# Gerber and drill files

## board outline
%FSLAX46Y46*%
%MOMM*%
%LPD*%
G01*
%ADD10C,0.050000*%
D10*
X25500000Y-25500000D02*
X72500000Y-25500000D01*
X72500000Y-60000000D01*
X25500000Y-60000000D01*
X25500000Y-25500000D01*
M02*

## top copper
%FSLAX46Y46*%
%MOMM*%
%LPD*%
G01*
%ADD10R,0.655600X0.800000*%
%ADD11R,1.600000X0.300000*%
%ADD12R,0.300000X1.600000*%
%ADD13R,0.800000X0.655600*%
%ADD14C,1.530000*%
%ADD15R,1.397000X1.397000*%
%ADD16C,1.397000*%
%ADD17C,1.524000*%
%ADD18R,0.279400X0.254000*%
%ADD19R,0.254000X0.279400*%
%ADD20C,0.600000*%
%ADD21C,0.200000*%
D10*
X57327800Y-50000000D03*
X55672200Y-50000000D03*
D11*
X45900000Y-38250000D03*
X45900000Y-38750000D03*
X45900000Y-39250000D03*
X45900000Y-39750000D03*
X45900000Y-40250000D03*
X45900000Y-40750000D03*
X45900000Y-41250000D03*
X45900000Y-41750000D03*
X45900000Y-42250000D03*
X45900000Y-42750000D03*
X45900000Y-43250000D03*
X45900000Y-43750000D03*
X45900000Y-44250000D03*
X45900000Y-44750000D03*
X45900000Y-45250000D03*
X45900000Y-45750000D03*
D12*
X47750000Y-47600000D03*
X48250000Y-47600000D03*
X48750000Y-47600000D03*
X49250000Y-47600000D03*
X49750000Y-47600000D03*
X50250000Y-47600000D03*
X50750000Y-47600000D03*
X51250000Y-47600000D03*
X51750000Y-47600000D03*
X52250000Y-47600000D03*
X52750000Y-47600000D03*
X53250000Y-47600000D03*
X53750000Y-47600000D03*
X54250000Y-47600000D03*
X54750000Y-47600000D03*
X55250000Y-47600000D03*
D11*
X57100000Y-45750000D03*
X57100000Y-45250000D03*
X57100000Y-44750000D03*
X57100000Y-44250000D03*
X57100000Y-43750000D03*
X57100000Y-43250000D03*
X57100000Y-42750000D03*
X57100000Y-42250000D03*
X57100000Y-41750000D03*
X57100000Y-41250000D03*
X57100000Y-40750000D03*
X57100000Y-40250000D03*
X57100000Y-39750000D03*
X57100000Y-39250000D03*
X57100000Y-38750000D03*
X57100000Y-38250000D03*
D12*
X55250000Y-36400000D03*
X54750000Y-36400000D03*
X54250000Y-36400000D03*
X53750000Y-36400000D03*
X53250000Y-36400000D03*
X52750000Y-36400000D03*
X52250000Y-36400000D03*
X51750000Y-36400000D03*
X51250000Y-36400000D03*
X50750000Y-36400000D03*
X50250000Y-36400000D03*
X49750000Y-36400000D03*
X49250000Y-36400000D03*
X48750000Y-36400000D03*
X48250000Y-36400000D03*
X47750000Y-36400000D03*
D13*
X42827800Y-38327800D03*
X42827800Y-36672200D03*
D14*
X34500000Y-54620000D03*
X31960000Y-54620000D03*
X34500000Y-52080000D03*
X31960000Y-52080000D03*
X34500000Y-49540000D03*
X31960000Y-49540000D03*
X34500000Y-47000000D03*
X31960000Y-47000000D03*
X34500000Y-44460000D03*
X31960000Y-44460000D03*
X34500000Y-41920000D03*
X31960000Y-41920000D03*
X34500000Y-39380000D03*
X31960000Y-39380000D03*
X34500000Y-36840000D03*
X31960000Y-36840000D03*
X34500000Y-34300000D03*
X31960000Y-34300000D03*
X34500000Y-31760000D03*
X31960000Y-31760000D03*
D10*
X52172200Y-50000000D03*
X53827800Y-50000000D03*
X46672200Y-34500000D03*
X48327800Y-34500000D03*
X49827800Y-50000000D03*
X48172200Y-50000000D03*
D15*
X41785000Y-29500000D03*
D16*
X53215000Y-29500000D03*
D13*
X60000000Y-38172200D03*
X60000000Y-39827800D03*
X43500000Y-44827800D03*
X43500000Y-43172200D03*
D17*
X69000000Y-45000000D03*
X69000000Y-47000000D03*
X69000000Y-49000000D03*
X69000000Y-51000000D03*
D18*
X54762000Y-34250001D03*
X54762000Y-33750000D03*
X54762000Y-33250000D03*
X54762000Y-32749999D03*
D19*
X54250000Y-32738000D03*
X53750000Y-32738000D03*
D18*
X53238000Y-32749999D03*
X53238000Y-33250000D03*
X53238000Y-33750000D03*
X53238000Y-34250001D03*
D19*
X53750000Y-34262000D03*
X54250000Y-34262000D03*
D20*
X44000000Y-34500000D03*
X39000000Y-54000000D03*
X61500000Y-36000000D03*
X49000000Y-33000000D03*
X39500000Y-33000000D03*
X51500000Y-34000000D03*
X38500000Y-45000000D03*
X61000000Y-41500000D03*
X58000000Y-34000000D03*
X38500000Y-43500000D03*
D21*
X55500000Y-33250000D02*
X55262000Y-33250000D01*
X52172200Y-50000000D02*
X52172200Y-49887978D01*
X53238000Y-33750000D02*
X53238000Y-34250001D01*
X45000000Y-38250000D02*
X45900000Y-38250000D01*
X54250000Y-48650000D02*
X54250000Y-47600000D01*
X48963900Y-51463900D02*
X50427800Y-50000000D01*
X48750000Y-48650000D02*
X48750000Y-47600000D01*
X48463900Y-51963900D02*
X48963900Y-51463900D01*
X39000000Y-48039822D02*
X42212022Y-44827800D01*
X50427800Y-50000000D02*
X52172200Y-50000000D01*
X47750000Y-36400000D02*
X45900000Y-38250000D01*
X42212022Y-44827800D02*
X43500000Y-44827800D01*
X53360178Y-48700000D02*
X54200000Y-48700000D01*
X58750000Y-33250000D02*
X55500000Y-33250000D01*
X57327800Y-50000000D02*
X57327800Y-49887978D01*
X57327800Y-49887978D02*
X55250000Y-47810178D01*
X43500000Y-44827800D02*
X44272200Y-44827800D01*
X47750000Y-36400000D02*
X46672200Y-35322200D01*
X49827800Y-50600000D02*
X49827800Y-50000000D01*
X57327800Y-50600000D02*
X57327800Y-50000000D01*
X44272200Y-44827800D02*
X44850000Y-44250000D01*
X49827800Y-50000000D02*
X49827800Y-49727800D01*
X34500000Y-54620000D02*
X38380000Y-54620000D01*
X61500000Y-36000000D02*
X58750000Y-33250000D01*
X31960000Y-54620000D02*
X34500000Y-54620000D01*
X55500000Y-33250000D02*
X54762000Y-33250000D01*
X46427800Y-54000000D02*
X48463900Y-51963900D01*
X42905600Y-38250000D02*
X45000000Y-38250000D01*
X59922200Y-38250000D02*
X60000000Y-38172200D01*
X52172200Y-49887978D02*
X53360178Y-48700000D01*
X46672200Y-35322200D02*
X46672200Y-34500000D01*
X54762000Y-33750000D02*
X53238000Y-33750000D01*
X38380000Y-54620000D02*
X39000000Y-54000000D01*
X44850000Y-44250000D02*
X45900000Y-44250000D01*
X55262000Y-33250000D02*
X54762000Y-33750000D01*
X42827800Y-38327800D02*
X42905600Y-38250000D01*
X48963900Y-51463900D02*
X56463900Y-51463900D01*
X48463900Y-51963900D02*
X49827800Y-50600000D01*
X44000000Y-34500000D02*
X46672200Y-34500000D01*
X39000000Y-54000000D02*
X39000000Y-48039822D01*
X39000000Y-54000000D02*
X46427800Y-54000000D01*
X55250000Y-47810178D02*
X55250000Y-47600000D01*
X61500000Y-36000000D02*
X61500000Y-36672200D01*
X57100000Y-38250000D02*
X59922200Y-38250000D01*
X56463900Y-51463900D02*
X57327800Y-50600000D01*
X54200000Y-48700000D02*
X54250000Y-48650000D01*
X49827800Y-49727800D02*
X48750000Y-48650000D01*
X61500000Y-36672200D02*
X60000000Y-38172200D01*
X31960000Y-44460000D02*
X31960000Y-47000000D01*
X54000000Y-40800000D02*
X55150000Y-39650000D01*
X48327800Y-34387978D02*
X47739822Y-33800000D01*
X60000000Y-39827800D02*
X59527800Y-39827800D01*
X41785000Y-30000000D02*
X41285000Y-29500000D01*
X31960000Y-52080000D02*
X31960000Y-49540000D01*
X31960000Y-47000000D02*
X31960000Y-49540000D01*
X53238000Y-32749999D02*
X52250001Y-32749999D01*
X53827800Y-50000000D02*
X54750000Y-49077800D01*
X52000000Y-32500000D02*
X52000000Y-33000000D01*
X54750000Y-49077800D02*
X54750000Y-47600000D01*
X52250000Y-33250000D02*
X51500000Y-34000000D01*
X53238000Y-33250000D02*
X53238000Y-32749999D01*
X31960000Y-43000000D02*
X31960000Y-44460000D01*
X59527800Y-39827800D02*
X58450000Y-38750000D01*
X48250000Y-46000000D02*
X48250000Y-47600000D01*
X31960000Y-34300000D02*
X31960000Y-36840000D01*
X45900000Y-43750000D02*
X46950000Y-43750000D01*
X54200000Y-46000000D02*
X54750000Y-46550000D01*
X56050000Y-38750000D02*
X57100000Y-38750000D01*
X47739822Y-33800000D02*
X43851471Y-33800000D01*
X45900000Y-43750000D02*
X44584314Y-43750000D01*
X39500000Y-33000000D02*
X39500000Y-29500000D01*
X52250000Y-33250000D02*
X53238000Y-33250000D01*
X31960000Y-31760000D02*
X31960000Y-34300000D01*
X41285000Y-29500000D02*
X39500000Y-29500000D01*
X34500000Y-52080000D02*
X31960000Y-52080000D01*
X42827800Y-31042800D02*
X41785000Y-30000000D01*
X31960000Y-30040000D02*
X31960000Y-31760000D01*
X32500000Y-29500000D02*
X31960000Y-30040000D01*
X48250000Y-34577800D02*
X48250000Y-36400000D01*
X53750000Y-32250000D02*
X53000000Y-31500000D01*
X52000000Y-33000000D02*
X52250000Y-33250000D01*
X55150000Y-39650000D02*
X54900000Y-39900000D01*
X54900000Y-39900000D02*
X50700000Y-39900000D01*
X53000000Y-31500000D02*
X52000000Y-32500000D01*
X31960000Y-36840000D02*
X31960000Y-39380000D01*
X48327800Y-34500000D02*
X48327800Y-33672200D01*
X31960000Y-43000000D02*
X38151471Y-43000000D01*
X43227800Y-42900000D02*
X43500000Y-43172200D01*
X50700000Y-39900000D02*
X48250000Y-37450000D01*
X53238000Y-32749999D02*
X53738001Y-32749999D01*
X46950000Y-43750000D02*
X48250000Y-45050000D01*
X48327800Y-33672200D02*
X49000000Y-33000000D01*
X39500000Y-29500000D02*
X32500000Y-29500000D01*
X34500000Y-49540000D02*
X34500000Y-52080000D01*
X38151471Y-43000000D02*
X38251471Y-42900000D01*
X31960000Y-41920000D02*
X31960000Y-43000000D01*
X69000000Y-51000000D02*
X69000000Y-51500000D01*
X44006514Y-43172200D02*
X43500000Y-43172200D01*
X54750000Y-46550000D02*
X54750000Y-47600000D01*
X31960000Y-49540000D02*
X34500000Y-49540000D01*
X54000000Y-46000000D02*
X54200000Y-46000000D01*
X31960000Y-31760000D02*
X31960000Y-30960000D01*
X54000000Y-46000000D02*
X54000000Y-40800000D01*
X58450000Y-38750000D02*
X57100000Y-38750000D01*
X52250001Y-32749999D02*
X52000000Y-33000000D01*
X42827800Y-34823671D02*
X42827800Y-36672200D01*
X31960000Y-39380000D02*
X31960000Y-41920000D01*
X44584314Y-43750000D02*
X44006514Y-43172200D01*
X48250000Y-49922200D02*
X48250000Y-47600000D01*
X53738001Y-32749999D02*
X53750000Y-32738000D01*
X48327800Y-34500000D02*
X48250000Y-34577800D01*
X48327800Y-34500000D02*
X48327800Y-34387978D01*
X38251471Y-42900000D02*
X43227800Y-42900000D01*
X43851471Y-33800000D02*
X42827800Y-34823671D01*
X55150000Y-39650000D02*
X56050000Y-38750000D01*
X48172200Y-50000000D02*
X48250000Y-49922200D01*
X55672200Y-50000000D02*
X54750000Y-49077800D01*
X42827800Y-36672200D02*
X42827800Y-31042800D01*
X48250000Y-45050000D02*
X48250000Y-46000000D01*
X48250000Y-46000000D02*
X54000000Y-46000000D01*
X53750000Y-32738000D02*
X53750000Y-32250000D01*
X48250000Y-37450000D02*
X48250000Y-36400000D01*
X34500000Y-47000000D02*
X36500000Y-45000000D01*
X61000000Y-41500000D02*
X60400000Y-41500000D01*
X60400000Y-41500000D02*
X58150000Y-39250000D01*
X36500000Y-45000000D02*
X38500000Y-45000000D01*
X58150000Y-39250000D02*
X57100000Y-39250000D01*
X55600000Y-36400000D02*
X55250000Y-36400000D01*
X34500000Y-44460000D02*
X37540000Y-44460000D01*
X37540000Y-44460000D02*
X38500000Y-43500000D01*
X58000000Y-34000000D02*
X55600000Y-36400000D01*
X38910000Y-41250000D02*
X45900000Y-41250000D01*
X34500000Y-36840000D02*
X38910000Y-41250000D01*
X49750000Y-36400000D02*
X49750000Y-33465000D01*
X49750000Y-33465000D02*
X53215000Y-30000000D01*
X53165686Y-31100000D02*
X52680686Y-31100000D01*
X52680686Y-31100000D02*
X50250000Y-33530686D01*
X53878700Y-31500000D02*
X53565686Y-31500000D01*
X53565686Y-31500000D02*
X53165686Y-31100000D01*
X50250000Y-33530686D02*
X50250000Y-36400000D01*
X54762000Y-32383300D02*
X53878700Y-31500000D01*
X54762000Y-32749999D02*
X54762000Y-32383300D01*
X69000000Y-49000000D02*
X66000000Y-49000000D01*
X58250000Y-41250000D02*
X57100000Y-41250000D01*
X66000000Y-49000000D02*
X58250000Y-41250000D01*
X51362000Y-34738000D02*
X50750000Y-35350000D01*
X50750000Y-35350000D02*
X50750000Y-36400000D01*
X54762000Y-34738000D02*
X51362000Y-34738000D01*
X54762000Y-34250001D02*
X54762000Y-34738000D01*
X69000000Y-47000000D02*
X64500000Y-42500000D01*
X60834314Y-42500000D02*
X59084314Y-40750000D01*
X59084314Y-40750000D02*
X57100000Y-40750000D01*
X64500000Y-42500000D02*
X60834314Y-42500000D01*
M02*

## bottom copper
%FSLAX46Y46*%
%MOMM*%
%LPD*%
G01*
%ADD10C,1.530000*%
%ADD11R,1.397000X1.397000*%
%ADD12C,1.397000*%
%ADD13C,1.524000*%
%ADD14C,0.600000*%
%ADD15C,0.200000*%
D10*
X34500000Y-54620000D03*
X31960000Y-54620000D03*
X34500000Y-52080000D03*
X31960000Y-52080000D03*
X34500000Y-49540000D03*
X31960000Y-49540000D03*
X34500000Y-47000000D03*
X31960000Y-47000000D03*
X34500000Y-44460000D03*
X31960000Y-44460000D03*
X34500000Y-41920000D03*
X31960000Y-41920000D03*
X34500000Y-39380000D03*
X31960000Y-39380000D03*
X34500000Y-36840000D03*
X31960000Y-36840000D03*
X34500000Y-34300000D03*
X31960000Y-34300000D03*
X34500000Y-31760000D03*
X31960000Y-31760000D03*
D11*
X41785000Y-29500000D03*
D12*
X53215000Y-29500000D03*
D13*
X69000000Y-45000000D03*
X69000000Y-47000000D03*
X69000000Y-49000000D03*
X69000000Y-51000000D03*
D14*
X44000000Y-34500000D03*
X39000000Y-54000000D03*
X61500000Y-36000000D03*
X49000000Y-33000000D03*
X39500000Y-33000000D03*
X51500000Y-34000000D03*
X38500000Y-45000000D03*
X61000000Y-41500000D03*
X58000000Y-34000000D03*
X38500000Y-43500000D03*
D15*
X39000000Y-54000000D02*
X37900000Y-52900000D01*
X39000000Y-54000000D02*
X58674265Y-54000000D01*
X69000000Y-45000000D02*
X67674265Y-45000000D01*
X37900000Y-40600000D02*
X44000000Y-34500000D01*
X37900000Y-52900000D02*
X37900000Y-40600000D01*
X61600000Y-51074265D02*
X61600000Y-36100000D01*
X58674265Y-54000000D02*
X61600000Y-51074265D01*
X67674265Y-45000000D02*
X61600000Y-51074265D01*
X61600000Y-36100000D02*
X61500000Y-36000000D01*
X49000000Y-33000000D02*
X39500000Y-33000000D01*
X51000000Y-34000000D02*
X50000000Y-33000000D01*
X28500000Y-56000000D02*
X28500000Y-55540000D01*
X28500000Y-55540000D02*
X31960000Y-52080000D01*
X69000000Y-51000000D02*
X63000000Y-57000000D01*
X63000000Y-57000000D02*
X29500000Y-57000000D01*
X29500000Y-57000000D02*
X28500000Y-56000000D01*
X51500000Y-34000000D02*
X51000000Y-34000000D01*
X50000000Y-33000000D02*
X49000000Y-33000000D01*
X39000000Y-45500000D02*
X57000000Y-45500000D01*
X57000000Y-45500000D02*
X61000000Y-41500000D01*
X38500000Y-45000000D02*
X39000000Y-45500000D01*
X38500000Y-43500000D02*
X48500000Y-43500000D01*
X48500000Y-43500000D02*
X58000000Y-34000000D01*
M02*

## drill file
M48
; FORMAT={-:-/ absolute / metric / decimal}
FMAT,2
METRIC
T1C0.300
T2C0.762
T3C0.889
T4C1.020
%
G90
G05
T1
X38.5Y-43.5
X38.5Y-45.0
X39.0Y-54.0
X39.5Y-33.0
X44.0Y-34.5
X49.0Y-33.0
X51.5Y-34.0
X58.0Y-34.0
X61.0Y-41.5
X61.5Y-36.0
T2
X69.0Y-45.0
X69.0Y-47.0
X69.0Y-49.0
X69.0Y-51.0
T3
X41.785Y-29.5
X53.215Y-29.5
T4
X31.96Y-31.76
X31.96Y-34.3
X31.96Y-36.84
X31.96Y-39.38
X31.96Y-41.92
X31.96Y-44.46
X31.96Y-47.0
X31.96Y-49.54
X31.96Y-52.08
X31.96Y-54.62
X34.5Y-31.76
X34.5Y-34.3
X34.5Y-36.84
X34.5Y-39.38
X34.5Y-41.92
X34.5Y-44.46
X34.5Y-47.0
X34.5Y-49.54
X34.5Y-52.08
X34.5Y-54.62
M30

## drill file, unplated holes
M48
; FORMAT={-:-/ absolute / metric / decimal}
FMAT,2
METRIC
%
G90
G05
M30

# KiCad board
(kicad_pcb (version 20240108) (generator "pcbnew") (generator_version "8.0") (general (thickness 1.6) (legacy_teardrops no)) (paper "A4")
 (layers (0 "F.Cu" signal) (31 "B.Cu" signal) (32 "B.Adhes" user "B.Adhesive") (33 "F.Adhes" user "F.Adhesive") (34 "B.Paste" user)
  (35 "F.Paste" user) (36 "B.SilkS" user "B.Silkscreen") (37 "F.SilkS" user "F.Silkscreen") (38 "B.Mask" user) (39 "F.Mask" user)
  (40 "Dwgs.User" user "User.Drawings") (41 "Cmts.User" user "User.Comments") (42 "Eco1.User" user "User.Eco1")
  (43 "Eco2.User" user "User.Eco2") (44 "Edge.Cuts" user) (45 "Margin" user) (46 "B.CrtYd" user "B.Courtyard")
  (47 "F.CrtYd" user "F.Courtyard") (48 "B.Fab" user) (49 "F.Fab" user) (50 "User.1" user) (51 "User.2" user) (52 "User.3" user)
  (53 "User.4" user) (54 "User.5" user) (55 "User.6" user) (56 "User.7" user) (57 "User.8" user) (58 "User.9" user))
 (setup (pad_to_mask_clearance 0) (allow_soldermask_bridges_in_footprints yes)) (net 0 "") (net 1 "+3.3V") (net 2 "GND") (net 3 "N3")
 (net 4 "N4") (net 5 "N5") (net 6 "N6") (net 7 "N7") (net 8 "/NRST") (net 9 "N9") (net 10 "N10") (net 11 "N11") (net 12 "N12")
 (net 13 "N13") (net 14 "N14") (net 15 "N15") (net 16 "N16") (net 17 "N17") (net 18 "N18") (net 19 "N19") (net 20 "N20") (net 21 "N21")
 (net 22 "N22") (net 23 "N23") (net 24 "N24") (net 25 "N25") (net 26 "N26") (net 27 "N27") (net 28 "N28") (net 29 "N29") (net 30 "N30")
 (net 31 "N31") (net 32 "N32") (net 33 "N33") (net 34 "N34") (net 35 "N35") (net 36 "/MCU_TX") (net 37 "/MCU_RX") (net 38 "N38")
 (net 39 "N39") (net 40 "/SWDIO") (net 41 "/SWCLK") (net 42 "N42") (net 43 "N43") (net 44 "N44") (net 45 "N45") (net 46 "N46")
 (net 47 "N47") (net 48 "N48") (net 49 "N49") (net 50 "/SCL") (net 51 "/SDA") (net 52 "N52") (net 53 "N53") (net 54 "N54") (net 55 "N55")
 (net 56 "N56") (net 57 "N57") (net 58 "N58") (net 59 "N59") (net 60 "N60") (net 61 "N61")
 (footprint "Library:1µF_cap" (layer "F.Cu") (at 56.5 50 180)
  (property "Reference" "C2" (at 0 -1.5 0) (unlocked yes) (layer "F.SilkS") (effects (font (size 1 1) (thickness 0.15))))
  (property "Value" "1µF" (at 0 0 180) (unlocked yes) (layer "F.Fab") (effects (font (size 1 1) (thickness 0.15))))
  (pad "1" smd rect (at -0.8278 0 180) (size 0.6556 0.8) (layers "F.Cu" "F.Paste" "F.Mask") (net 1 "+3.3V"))
  (pad "2" smd rect (at 0.8278 0 180) (size 0.6556 0.8) (layers "F.Cu" "F.Paste" "F.Mask") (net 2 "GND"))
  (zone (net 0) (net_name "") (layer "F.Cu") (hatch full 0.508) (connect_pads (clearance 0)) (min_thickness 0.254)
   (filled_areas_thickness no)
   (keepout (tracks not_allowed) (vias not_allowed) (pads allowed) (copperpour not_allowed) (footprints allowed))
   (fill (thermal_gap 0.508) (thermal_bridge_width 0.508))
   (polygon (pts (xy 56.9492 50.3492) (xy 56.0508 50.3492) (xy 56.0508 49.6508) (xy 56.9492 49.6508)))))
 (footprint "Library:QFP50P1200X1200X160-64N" (layer "F.Cu") (at 51.5 42)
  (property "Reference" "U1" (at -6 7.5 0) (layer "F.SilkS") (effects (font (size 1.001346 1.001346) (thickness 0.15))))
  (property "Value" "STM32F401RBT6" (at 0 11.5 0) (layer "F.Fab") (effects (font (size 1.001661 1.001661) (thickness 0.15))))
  (pad "1" smd rect (at -5.6 -3.75) (size 1.6 0.3) (layers "F.Cu" "F.Paste" "F.Mask") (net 1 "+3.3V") (solder_mask_margin 0.102))
  (pad "2" smd rect (at -5.6 -3.25) (size 1.6 0.3) (layers "F.Cu" "F.Paste" "F.Mask") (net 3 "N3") (solder_mask_margin 0.102))
  (pad "3" smd rect (at -5.6 -2.75) (size 1.6 0.3) (layers "F.Cu" "F.Paste" "F.Mask") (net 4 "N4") (solder_mask_margin 0.102))
  (pad "4" smd rect (at -5.6 -2.25) (size 1.6 0.3) (layers "F.Cu" "F.Paste" "F.Mask") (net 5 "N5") (solder_mask_margin 0.102))
  (pad "5" smd rect (at -5.6 -1.75) (size 1.6 0.3) (layers "F.Cu" "F.Paste" "F.Mask") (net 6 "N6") (solder_mask_margin 0.102))
  (pad "6" smd rect (at -5.6 -1.25) (size 1.6 0.3) (layers "F.Cu" "F.Paste" "F.Mask") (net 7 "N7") (solder_mask_margin 0.102))
  (pad "7" smd rect (at -5.6 -0.75) (size 1.6 0.3) (layers "F.Cu" "F.Paste" "F.Mask") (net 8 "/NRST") (solder_mask_margin 0.102))
  (pad "8" smd rect (at -5.6 -0.25) (size 1.6 0.3) (layers "F.Cu" "F.Paste" "F.Mask") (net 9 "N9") (solder_mask_margin 0.102))
  (pad "9" smd rect (at -5.6 0.25) (size 1.6 0.3) (layers "F.Cu" "F.Paste" "F.Mask") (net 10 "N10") (solder_mask_margin 0.102))
  (pad "10" smd rect (at -5.6 0.75) (size 1.6 0.3) (layers "F.Cu" "F.Paste" "F.Mask") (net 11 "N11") (solder_mask_margin 0.102))
  (pad "11" smd rect (at -5.6 1.25) (size 1.6 0.3) (layers "F.Cu" "F.Paste" "F.Mask") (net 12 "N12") (solder_mask_margin 0.102))
  (pad "12" smd rect (at -5.6 1.75) (size 1.6 0.3) (layers "F.Cu" "F.Paste" "F.Mask") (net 2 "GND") (solder_mask_margin 0.102))
  (pad "13" smd rect (at -5.6 2.25) (size 1.6 0.3) (layers "F.Cu" "F.Paste" "F.Mask") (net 1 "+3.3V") (solder_mask_margin 0.102))
  (pad "14" smd rect (at -5.6 2.75) (size 1.6 0.3) (layers "F.Cu" "F.Paste" "F.Mask") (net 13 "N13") (solder_mask_margin 0.102))
  (pad "15" smd rect (at -5.6 3.25) (size 1.6 0.3) (layers "F.Cu" "F.Paste" "F.Mask") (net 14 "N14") (solder_mask_margin 0.102))
  (pad "16" smd rect (at -5.6 3.75) (size 1.6 0.3) (layers "F.Cu" "F.Paste" "F.Mask") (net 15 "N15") (solder_mask_margin 0.102))
  (pad "17" smd rect (at -3.75 5.6) (size 0.3 1.6) (layers "F.Cu" "F.Paste" "F.Mask") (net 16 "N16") (solder_mask_margin 0.102))
  (pad "18" smd rect (at -3.25 5.6) (size 0.3 1.6) (layers "F.Cu" "F.Paste" "F.Mask") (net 2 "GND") (solder_mask_margin 0.102))
  (pad "19" smd rect (at -2.75 5.6) (size 0.3 1.6) (layers "F.Cu" "F.Paste" "F.Mask") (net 1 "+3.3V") (solder_mask_margin 0.102))
  (pad "20" smd rect (at -2.25 5.6) (size 0.3 1.6) (layers "F.Cu" "F.Paste" "F.Mask") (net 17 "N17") (solder_mask_margin 0.102))
  (pad "21" smd rect (at -1.75 5.6) (size 0.3 1.6) (layers "F.Cu" "F.Paste" "F.Mask") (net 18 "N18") (solder_mask_margin 0.102))
  (pad "22" smd rect (at -1.25 5.6) (size 0.3 1.6) (layers "F.Cu" "F.Paste" "F.Mask") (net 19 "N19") (solder_mask_margin 0.102))
  (pad "23" smd rect (at -0.75 5.6) (size 0.3 1.6) (layers "F.Cu" "F.Paste" "F.Mask") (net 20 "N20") (solder_mask_margin 0.102))
  (pad "24" smd rect (at -0.25 5.6) (size 0.3 1.6) (layers "F.Cu" "F.Paste" "F.Mask") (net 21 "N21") (solder_mask_margin 0.102))
  (pad "25" smd rect (at 0.25 5.6) (size 0.3 1.6) (layers "F.Cu" "F.Paste" "F.Mask") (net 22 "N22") (solder_mask_margin 0.102))
  (pad "26" smd rect (at 0.75 5.6) (size 0.3 1.6) (layers "F.Cu" "F.Paste" "F.Mask") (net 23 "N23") (solder_mask_margin 0.102))
  (pad "27" smd rect (at 1.25 5.6) (size 0.3 1.6) (layers "F.Cu" "F.Paste" "F.Mask") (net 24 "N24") (solder_mask_margin 0.102))
  (pad "28" smd rect (at 1.75 5.6) (size 0.3 1.6) (layers "F.Cu" "F.Paste" "F.Mask") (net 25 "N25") (solder_mask_margin 0.102))
  (pad "29" smd rect (at 2.25 5.6) (size 0.3 1.6) (layers "F.Cu" "F.Paste" "F.Mask") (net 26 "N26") (solder_mask_margin 0.102))
  (pad "30" smd rect (at 2.75 5.6) (size 0.3 1.6) (layers "F.Cu" "F.Paste" "F.Mask") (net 1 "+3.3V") (solder_mask_margin 0.102))
  (pad "31" smd rect (at 3.25 5.6) (size 0.3 1.6) (layers "F.Cu" "F.Paste" "F.Mask") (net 2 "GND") (solder_mask_margin 0.102))
  (pad "32" smd rect (at 3.75 5.6) (size 0.3 1.6) (layers "F.Cu" "F.Paste" "F.Mask") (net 1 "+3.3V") (solder_mask_margin 0.102))
  (pad "33" smd rect (at 5.6 3.75) (size 1.6 0.3) (layers "F.Cu" "F.Paste" "F.Mask") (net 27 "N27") (solder_mask_margin 0.102))
  (pad "34" smd rect (at 5.6 3.25) (size 1.6 0.3) (layers "F.Cu" "F.Paste" "F.Mask") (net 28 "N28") (solder_mask_margin 0.102))
  (pad "35" smd rect (at 5.6 2.75) (size 1.6 0.3) (layers "F.Cu" "F.Paste" "F.Mask") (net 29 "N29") (solder_mask_margin 0.102))
  (pad "36" smd rect (at 5.6 2.25) (size 1.6 0.3) (layers "F.Cu" "F.Paste" "F.Mask") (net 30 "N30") (solder_mask_margin 0.102))
  (pad "37" smd rect (at 5.6 1.75) (size 1.6 0.3) (layers "F.Cu" "F.Paste" "F.Mask") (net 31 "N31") (solder_mask_margin 0.102))
  (pad "38" smd rect (at 5.6 1.25) (size 1.6 0.3) (layers "F.Cu" "F.Paste" "F.Mask") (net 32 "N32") (solder_mask_margin 0.102))
  (pad "39" smd rect (at 5.6 0.75) (size 1.6 0.3) (layers "F.Cu" "F.Paste" "F.Mask") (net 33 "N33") (solder_mask_margin 0.102))
  (pad "40" smd rect (at 5.6 0.25) (size 1.6 0.3) (layers "F.Cu" "F.Paste" "F.Mask") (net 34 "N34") (solder_mask_margin 0.102))
  (pad "41" smd rect (at 5.6 -0.25) (size 1.6 0.3) (layers "F.Cu" "F.Paste" "F.Mask") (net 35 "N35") (solder_mask_margin 0.102))
  (pad "42" smd rect (at 5.6 -0.75) (size 1.6 0.3) (layers "F.Cu" "F.Paste" "F.Mask") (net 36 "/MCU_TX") (solder_mask_margin 0.102))
  (pad "43" smd rect (at 5.6 -1.25) (size 1.6 0.3) (layers "F.Cu" "F.Paste" "F.Mask") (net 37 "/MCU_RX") (solder_mask_margin 0.102))
  (pad "44" smd rect (at 5.6 -1.75) (size 1.6 0.3) (layers "F.Cu" "F.Paste" "F.Mask") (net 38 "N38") (solder_mask_margin 0.102))
  (pad "45" smd rect (at 5.6 -2.25) (size 1.6 0.3) (layers "F.Cu" "F.Paste" "F.Mask") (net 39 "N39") (solder_mask_margin 0.102))
  (pad "46" smd rect (at 5.6 -2.75) (size 1.6 0.3) (layers "F.Cu" "F.Paste" "F.Mask") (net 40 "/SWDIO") (solder_mask_margin 0.102))
  (pad "47" smd rect (at 5.6 -3.25) (size 1.6 0.3) (layers "F.Cu" "F.Paste" "F.Mask") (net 2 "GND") (solder_mask_margin 0.102))
  (pad "48" smd rect (at 5.6 -3.75) (size 1.6 0.3) (layers "F.Cu" "F.Paste" "F.Mask") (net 1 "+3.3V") (solder_mask_margin 0.102))
  (pad "49" smd rect (at 3.75 -5.6) (size 0.3 1.6) (layers "F.Cu" "F.Paste" "F.Mask") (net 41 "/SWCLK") (solder_mask_margin 0.102))
  (pad "50" smd rect (at 3.25 -5.6) (size 0.3 1.6) (layers "F.Cu" "F.Paste" "F.Mask") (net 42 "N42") (solder_mask_margin 0.102))
  (pad "51" smd rect (at 2.75 -5.6) (size 0.3 1.6) (layers "F.Cu" "F.Paste" "F.Mask") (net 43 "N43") (solder_mask_margin 0.102))
  (pad "52" smd rect (at 2.25 -5.6) (size 0.3 1.6) (layers "F.Cu" "F.Paste" "F.Mask") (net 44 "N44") (solder_mask_margin 0.102))
  (pad "53" smd rect (at 1.75 -5.6) (size 0.3 1.6) (layers "F.Cu" "F.Paste" "F.Mask") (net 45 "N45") (solder_mask_margin 0.102))
  (pad "54" smd rect (at 1.25 -5.6) (size 0.3 1.6) (layers "F.Cu" "F.Paste" "F.Mask") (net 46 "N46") (solder_mask_margin 0.102))
  (pad "55" smd rect (at 0.75 -5.6) (size 0.3 1.6) (layers "F.Cu" "F.Paste" "F.Mask") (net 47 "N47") (solder_mask_margin 0.102))
  (pad "56" smd rect (at 0.25 -5.6) (size 0.3 1.6) (layers "F.Cu" "F.Paste" "F.Mask") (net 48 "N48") (solder_mask_margin 0.102))
  (pad "57" smd rect (at -0.25 -5.6) (size 0.3 1.6) (layers "F.Cu" "F.Paste" "F.Mask") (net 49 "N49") (solder_mask_margin 0.102))
  (pad "58" smd rect (at -0.75 -5.6) (size 0.3 1.6) (layers "F.Cu" "F.Paste" "F.Mask") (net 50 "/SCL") (solder_mask_margin 0.102))
  (pad "59" smd rect (at -1.25 -5.6) (size 0.3 1.6) (layers "F.Cu" "F.Paste" "F.Mask") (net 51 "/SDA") (solder_mask_margin 0.102))
  (pad "60" smd rect (at -1.75 -5.6) (size 0.3 1.6) (layers "F.Cu" "F.Paste" "F.Mask") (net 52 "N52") (solder_mask_margin 0.102))
  (pad "61" smd rect (at -2.25 -5.6) (size 0.3 1.6) (layers "F.Cu" "F.Paste" "F.Mask") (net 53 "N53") (solder_mask_margin 0.102))
  (pad "62" smd rect (at -2.75 -5.6) (size 0.3 1.6) (layers "F.Cu" "F.Paste" "F.Mask") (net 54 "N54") (solder_mask_margin 0.102))
  (pad "63" smd rect (at -3.25 -5.6) (size 0.3 1.6) (layers "F.Cu" "F.Paste" "F.Mask") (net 2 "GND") (solder_mask_margin 0.102))
  (pad "64" smd rect (at -3.75 -5.6) (size 0.3 1.6) (layers "F.Cu" "F.Paste" "F.Mask") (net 1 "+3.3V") (solder_mask_margin 0.102)))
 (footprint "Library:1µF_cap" (layer "F.Cu") (at 42.8278 37.5 90)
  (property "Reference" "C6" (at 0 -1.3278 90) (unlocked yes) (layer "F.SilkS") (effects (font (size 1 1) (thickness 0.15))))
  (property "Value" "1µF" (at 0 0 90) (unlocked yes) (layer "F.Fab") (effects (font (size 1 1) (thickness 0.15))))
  (pad "1" smd rect (at -0.8278 0 90) (size 0.6556 0.8) (layers "F.Cu" "F.Paste" "F.Mask") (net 1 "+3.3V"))
  (pad "2" smd rect (at 0.8278 0 90) (size 0.6556 0.8) (layers "F.Cu" "F.Paste" "F.Mask") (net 2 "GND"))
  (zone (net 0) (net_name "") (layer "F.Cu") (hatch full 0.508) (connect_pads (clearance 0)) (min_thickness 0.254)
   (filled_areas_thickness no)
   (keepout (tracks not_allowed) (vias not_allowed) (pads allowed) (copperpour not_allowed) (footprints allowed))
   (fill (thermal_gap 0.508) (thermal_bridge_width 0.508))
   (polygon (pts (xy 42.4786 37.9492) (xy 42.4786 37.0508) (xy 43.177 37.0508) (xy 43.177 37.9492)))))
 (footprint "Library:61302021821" (layer "F.Cu") (at 33.23 43.19 90)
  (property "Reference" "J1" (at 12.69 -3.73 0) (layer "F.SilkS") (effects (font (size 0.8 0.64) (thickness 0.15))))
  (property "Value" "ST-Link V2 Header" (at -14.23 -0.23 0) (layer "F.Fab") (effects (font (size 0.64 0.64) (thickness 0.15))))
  (pad "1" thru_hole circle (at -11.43 1.27 90) (size 1.53 1.53) (drill 1.02) (layers "*.Cu" "*.Mask") (remove_unused_layers no)
   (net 1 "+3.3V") (solder_mask_margin 0.102))
  (pad "2" thru_hole circle (at -11.43 -1.27 90) (size 1.53 1.53) (drill 1.02) (layers "*.Cu" "*.Mask") (remove_unused_layers no)
   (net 1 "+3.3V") (solder_mask_margin 0.102))
  (pad "3" thru_hole circle (at -8.89 1.27 90) (size 1.53 1.53) (drill 1.02) (layers "*.Cu" "*.Mask") (remove_unused_layers no)
   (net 2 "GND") (solder_mask_margin 0.102))
  (pad "4" thru_hole circle (at -8.89 -1.27 90) (size 1.53 1.53) (drill 1.02) (layers "*.Cu" "*.Mask") (remove_unused_layers no)
   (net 2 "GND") (solder_mask_margin 0.102))
  (pad "5" thru_hole circle (at -6.35 1.27 90) (size 1.53 1.53) (drill 1.02) (layers "*.Cu" "*.Mask") (remove_unused_layers no)
   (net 2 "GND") (solder_mask_margin 0.102))
  (pad "6" thru_hole circle (at -6.35 -1.27 90) (size 1.53 1.53) (drill 1.02) (layers "*.Cu" "*.Mask") (remove_unused_layers no)
   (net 2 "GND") (solder_mask_margin 0.102))
  (pad "7" thru_hole circle (at -3.81 1.27 90) (size 1.53 1.53) (drill 1.02) (layers "*.Cu" "*.Mask") (remove_unused_layers no)
   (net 40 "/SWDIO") (solder_mask_margin 0.102))
  (pad "8" thru_hole circle (at -3.81 -1.27 90) (size 1.53 1.53) (drill 1.02) (layers "*.Cu" "*.Mask") (remove_unused_layers no)
   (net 2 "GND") (solder_mask_margin 0.102))
  (pad "9" thru_hole circle (at -1.27 1.27 90) (size 1.53 1.53) (drill 1.02) (layers "*.Cu" "*.Mask") (remove_unused_layers no)
   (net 41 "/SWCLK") (solder_mask_margin 0.102))
  (pad "10" thru_hole circle (at -1.27 -1.27 90) (size 1.53 1.53) (drill 1.02) (layers "*.Cu" "*.Mask") (remove_unused_layers no)
   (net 2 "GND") (solder_mask_margin 0.102))
  (pad "11" thru_hole circle (at 1.27 1.27 90) (size 1.53 1.53) (drill 1.02) (layers "*.Cu" "*.Mask") (remove_unused_layers no)
   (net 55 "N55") (solder_mask_margin 0.102))
  (pad "12" thru_hole circle (at 1.27 -1.27 90) (size 1.53 1.53) (drill 1.02) (layers "*.Cu" "*.Mask") (remove_unused_layers no)
   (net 2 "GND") (solder_mask_margin 0.102))
  (pad "13" thru_hole circle (at 3.81 1.27 90) (size 1.53 1.53) (drill 1.02) (layers "*.Cu" "*.Mask") (remove_unused_layers no)
   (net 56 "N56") (solder_mask_margin 0.102))
  (pad "14" thru_hole circle (at 3.81 -1.27 90) (size 1.53 1.53) (drill 1.02) (layers "*.Cu" "*.Mask") (remove_unused_layers no)
   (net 2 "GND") (solder_mask_margin 0.102))
  (pad "15" thru_hole circle (at 6.35 1.27 90) (size 1.53 1.53) (drill 1.02) (layers "*.Cu" "*.Mask") (remove_unused_layers no)
   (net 8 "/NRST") (solder_mask_margin 0.102))
  (pad "16" thru_hole circle (at 6.35 -1.27 90) (size 1.53 1.53) (drill 1.02) (layers "*.Cu" "*.Mask") (remove_unused_layers no)
   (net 2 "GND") (solder_mask_margin 0.102))
  (pad "17" thru_hole circle (at 8.89 1.27 90) (size 1.53 1.53) (drill 1.02) (layers "*.Cu" "*.Mask") (remove_unused_layers no)
   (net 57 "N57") (solder_mask_margin 0.102))
  (pad "18" thru_hole circle (at 8.89 -1.27 90) (size 1.53 1.53) (drill 1.02) (layers "*.Cu" "*.Mask") (remove_unused_layers no)
   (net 2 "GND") (solder_mask_margin 0.102))
  (pad "19" thru_hole circle (at 11.43 1.27 90) (size 1.53 1.53) (drill 1.02) (layers "*.Cu" "*.Mask") (remove_unused_layers no)
   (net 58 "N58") (solder_mask_margin 0.102))
  (pad "20" thru_hole circle (at 11.43 -1.27 90) (size 1.53 1.53) (drill 1.02) (layers "*.Cu" "*.Mask") (remove_unused_layers no)
   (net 2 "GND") (solder_mask_margin 0.102)))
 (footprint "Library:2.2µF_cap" (layer "F.Cu") (at 53 50)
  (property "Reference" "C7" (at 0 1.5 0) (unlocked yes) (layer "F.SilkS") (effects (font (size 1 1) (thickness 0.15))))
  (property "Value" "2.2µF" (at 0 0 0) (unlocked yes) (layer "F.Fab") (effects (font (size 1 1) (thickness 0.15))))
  (pad "1" smd rect (at -0.8278 0) (size 0.6556 0.8) (layers "F.Cu" "F.Paste" "F.Mask") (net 1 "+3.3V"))
  (pad "2" smd rect (at 0.8278 0) (size 0.6556 0.8) (layers "F.Cu" "F.Paste" "F.Mask") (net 2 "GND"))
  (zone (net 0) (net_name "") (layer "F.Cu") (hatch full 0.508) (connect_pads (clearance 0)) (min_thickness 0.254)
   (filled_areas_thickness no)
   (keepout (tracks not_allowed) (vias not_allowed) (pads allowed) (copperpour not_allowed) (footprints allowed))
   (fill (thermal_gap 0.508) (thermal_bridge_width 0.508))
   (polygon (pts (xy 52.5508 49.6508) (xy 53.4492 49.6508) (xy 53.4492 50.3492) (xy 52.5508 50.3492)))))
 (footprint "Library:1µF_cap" (layer "F.Cu") (at 47.5 34.5)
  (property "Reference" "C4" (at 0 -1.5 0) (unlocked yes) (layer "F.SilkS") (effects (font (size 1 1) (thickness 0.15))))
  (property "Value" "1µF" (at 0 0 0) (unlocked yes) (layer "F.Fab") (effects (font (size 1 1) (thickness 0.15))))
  (pad "1" smd rect (at -0.8278 0) (size 0.6556 0.8) (layers "F.Cu" "F.Paste" "F.Mask") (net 1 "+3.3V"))
  (pad "2" smd rect (at 0.8278 0) (size 0.6556 0.8) (layers "F.Cu" "F.Paste" "F.Mask") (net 2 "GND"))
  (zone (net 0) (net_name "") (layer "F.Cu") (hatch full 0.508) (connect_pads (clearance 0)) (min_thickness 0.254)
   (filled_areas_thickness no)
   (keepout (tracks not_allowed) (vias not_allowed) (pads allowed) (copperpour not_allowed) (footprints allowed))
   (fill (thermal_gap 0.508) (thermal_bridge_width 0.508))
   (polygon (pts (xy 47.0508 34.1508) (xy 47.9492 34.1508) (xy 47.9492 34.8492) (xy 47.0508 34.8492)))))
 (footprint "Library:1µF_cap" (layer "F.Cu") (at 49 50 180)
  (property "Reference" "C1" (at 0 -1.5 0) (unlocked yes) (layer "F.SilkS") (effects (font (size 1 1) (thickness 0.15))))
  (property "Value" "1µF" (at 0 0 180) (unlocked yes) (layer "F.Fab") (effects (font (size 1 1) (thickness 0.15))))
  (pad "1" smd rect (at -0.8278 0 180) (size 0.6556 0.8) (layers "F.Cu" "F.Paste" "F.Mask") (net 1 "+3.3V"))
  (pad "2" smd rect (at 0.8278 0 180) (size 0.6556 0.8) (layers "F.Cu" "F.Paste" "F.Mask") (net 2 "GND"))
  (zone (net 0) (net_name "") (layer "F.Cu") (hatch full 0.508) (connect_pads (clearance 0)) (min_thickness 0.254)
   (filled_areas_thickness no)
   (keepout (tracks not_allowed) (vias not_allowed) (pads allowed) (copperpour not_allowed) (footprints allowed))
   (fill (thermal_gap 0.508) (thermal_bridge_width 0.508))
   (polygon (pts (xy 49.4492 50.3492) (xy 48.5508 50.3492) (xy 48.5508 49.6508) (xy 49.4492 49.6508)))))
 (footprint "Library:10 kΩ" (layer "F.Cu") (at 41.785 29.5)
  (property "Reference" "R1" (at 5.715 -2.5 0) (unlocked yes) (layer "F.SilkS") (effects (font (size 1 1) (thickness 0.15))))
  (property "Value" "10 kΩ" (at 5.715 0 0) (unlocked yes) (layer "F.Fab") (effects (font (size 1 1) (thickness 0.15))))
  (pad "1" thru_hole rect (at 0 0) (size 1.397 1.397) (drill 0.889) (layers "*.Cu" "*.Mask") (remove_unused_layers no) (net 2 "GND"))
  (pad "2" thru_hole circle (at 11.43 0) (size 1.397 1.397) (drill 0.889) (layers "*.Cu" "*.Mask") (remove_unused_layers no) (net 52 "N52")))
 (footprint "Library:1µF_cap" (layer "F.Cu") (at 60 39 -90)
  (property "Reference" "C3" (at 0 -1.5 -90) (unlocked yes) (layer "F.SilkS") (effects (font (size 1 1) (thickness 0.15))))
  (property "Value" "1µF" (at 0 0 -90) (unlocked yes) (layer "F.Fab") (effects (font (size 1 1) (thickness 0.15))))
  (pad "1" smd rect (at -0.8278 0 270) (size 0.6556 0.8) (layers "F.Cu" "F.Paste" "F.Mask") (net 1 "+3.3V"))
  (pad "2" smd rect (at 0.8278 0 270) (size 0.6556 0.8) (layers "F.Cu" "F.Paste" "F.Mask") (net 2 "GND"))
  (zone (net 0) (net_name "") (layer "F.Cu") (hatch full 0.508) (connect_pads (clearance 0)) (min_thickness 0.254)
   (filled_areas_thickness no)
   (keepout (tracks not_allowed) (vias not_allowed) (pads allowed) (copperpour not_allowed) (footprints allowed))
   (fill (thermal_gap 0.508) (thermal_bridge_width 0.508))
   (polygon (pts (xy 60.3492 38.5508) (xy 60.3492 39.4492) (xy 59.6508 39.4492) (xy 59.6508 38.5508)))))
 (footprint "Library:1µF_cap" (layer "F.Cu") (at 43.5 44 90)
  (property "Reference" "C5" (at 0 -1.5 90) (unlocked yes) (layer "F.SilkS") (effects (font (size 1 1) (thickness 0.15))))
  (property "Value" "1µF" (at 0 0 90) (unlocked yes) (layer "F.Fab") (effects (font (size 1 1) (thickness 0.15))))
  (pad "1" smd rect (at -0.8278 0 90) (size 0.6556 0.8) (layers "F.Cu" "F.Paste" "F.Mask") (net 1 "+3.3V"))
  (pad "2" smd rect (at 0.8278 0 90) (size 0.6556 0.8) (layers "F.Cu" "F.Paste" "F.Mask") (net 2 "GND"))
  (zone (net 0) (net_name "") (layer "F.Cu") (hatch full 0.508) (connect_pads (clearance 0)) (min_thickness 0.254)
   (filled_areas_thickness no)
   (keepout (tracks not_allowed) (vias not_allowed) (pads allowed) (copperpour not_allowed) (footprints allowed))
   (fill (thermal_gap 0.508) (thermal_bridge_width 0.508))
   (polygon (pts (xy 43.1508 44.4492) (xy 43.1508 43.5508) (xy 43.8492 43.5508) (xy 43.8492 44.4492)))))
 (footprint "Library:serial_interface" (layer "F.Cu") (at 69 48 -90)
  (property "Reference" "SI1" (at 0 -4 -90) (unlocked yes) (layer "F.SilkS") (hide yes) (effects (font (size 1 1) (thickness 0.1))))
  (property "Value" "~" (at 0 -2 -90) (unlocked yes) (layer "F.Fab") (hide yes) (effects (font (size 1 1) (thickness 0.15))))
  (pad "1" thru_hole circle (at -3 0 270) (size 1.524 1.524) (drill 0.762) (layers "*.Cu" "*.Mask") (remove_unused_layers no)
   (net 1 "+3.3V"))
  (pad "2" thru_hole circle (at -1 0 270) (size 1.524 1.524) (drill 0.762) (layers "*.Cu" "*.Mask") (remove_unused_layers no)
   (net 37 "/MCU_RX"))
  (pad "3" thru_hole circle (at 1 0 270) (size 1.524 1.524) (drill 0.762) (layers "*.Cu" "*.Mask") (remove_unused_layers no)
   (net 36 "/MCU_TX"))
  (pad "4" thru_hole circle (at 3 0 270) (size 1.524 1.524) (drill 0.762) (layers "*.Cu" "*.Mask") (remove_unused_layers no) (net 2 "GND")))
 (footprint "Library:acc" (layer "F.Cu") (at 54 33.5 180)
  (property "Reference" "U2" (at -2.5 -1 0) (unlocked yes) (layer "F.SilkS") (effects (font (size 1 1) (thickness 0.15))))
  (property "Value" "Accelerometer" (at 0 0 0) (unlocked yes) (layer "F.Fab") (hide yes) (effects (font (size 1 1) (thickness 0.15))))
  (pad "1" smd rect (at -0.762 -0.750001 270) (size 0.254 0.2794) (layers "F.Cu" "F.Paste" "F.Mask") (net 50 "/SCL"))
  (pad "2" smd rect (at -0.762 -0.25 270) (size 0.254 0.2794) (layers "F.Cu" "F.Paste" "F.Mask") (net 1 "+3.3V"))
  (pad "3" smd rect (at -0.762 0.25 270) (size 0.254 0.2794) (layers "F.Cu" "F.Paste" "F.Mask") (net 1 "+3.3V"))
  (pad "4" smd rect (at -0.762 0.750001 270) (size 0.254 0.2794) (layers "F.Cu" "F.Paste" "F.Mask") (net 51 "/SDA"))
  (pad "5" smd rect (at -0.25 0.762 180) (size 0.254 0.2794) (layers "F.Cu" "F.Paste" "F.Mask") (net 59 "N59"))
  (pad "6" smd rect (at 0.25 0.762 180) (size 0.254 0.2794) (layers "F.Cu" "F.Paste" "F.Mask") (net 2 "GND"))
  (pad "7" smd rect (at 0.762 0.750001 270) (size 0.254 0.2794) (layers "F.Cu" "F.Paste" "F.Mask") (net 2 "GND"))
  (pad "8" smd rect (at 0.762 0.25 270) (size 0.254 0.2794) (layers "F.Cu" "F.Paste" "F.Mask") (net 2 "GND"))
  (pad "9" smd rect (at 0.762 -0.25 270) (size 0.254 0.2794) (layers "F.Cu" "F.Paste" "F.Mask") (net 1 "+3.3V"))
  (pad "10" smd rect (at 0.762 -0.750001 270) (size 0.254 0.2794) (layers "F.Cu" "F.Paste" "F.Mask") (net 1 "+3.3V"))
  (pad "11" smd rect (at 0.25 -0.762 180) (size 0.254 0.2794) (layers "F.Cu" "F.Paste" "F.Mask") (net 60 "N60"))
  (pad "12" smd rect (at -0.25 -0.762 180) (size 0.254 0.2794) (layers "F.Cu" "F.Paste" "F.Mask") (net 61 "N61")))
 (gr_rect (start 25.5 25.5) (end 72.5 60) (stroke (width 0.05) (type default)) (fill none) (layer "Edge.Cuts"))
 (segment (start 55.5 33.25) (end 55.262 33.25) (width 0.2) (layer "F.Cu") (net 1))
 (segment (start 52.1722 50) (end 52.1722 49.887978) (width 0.2) (layer "F.Cu") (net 1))
 (segment (start 53.238 33.75) (end 53.238 34.250001) (width 0.2) (layer "F.Cu") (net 1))
 (segment (start 45 38.25) (end 45.9 38.25) (width 0.2) (layer "F.Cu") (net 1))
 (segment (start 54.25 48.65) (end 54.25 47.6) (width 0.2) (layer "F.Cu") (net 1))
 (segment (start 48.9639 51.4639) (end 50.4278 50) (width 0.2) (layer "F.Cu") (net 1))
 (segment (start 48.75 48.65) (end 48.75 47.6) (width 0.2) (layer "F.Cu") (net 1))
 (segment (start 48.4639 51.9639) (end 48.9639 51.4639) (width 0.2) (layer "F.Cu") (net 1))
 (segment (start 39 48.039822) (end 42.212022 44.8278) (width 0.2) (layer "F.Cu") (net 1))
 (segment (start 50.4278 50) (end 52.1722 50) (width 0.2) (layer "F.Cu") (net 1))
 (segment (start 47.75 36.4) (end 45.9 38.25) (width 0.2) (layer "F.Cu") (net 1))
 (segment (start 42.212022 44.8278) (end 43.5 44.8278) (width 0.2) (layer "F.Cu") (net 1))
 (segment (start 53.360178 48.7) (end 54.2 48.7) (width 0.2) (layer "F.Cu") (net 1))
 (segment (start 58.75 33.25) (end 55.5 33.25) (width 0.2) (layer "F.Cu") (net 1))
 (segment (start 57.3278 50) (end 57.3278 49.887978) (width 0.2) (layer "F.Cu") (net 1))
 (segment (start 57.3278 49.887978) (end 55.25 47.810178) (width 0.2) (layer "F.Cu") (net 1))
 (segment (start 43.5 44.8278) (end 44.2722 44.8278) (width 0.2) (layer "F.Cu") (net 1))
 (segment (start 47.75 36.4) (end 46.6722 35.3222) (width 0.2) (layer "F.Cu") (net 1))
 (segment (start 49.8278 50.6) (end 49.8278 50) (width 0.2) (layer "F.Cu") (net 1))
 (segment (start 57.3278 50.6) (end 57.3278 50) (width 0.2) (layer "F.Cu") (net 1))
 (segment (start 44.2722 44.8278) (end 44.85 44.25) (width 0.2) (layer "F.Cu") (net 1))
 (segment (start 49.8278 50) (end 49.8278 49.7278) (width 0.2) (layer "F.Cu") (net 1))
 (segment (start 34.5 54.62) (end 38.38 54.62) (width 0.2) (layer "F.Cu") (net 1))
 (segment (start 61.5 36) (end 58.75 33.25) (width 0.2) (layer "F.Cu") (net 1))
 (segment (start 31.96 54.62) (end 34.5 54.62) (width 0.2) (layer "F.Cu") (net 1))
 (segment (start 55.5 33.25) (end 54.762 33.25) (width 0.2) (layer "F.Cu") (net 1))
 (segment (start 46.4278 54) (end 48.4639 51.9639) (width 0.2) (layer "F.Cu") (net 1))
 (segment (start 42.9056 38.25) (end 45 38.25) (width 0.2) (layer "F.Cu") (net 1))
 (segment (start 59.9222 38.25) (end 60 38.1722) (width 0.2) (layer "F.Cu") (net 1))
 (segment (start 52.1722 49.887978) (end 53.360178 48.7) (width 0.2) (layer "F.Cu") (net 1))
 (segment (start 46.6722 35.3222) (end 46.6722 34.5) (width 0.2) (layer "F.Cu") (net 1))
 (segment (start 54.762 33.75) (end 53.238 33.75) (width 0.2) (layer "F.Cu") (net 1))
 (segment (start 38.38 54.62) (end 39 54) (width 0.2) (layer "F.Cu") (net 1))
 (segment (start 44.85 44.25) (end 45.9 44.25) (width 0.2) (layer "F.Cu") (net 1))
 (segment (start 55.262 33.25) (end 54.762 33.75) (width 0.2) (layer "F.Cu") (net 1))
 (segment (start 42.8278 38.3278) (end 42.9056 38.25) (width 0.2) (layer "F.Cu") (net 1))
 (segment (start 48.9639 51.4639) (end 56.4639 51.4639) (width 0.2) (layer "F.Cu") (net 1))
 (segment (start 48.4639 51.9639) (end 49.8278 50.6) (width 0.2) (layer "F.Cu") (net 1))
 (segment (start 44 34.5) (end 46.6722 34.5) (width 0.2) (layer "F.Cu") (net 1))
 (segment (start 39 54) (end 39 48.039822) (width 0.2) (layer "F.Cu") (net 1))
 (segment (start 39 54) (end 46.4278 54) (width 0.2) (layer "F.Cu") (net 1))
 (segment (start 55.25 47.810178) (end 55.25 47.6) (width 0.2) (layer "F.Cu") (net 1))
 (segment (start 61.5 36) (end 61.5 36.6722) (width 0.2) (layer "F.Cu") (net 1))
 (segment (start 57.1 38.25) (end 59.9222 38.25) (width 0.2) (layer "F.Cu") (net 1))
 (segment (start 56.4639 51.4639) (end 57.3278 50.6) (width 0.2) (layer "F.Cu") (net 1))
 (segment (start 54.2 48.7) (end 54.25 48.65) (width 0.2) (layer "F.Cu") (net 1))
 (segment (start 49.8278 49.7278) (end 48.75 48.65) (width 0.2) (layer "F.Cu") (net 1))
 (segment (start 61.5 36.6722) (end 60 38.1722) (width 0.2) (layer "F.Cu") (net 1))
 (via (at 44 34.5) (size 0.6) (drill 0.3) (layers "F.Cu" "B.Cu") (free yes) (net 1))
 (via (at 39 54) (size 0.6) (drill 0.3) (layers "F.Cu" "B.Cu") (free yes) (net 1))
 (via (at 61.5 36) (size 0.6) (drill 0.3) (layers "F.Cu" "B.Cu") (free yes) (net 1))
 (segment (start 39 54) (end 37.9 52.9) (width 0.2) (layer "B.Cu") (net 1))
 (segment (start 39 54) (end 58.674265 54) (width 0.2) (layer "B.Cu") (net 1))
 (segment (start 69 45) (end 67.674265 45) (width 0.2) (layer "B.Cu") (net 1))
 (segment (start 37.9 40.6) (end 44 34.5) (width 0.2) (layer "B.Cu") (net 1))
 (segment (start 37.9 52.9) (end 37.9 40.6) (width 0.2) (layer "B.Cu") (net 1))
 (segment (start 61.6 51.074265) (end 61.6 36.1) (width 0.2) (layer "B.Cu") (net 1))
 (segment (start 58.674265 54) (end 61.6 51.074265) (width 0.2) (layer "B.Cu") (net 1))
 (segment (start 67.674265 45) (end 61.6 51.074265) (width 0.2) (layer "B.Cu") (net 1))
 (segment (start 61.6 36.1) (end 61.5 36) (width 0.2) (layer "B.Cu") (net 1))
 (segment (start 31.96 44.46) (end 31.96 47) (width 0.2) (layer "F.Cu") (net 2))
 (segment (start 54 40.8) (end 55.15 39.65) (width 0.2) (layer "F.Cu") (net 2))
 (segment (start 48.3278 34.387978) (end 47.739822 33.8) (width 0.2) (layer "F.Cu") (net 2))
 (segment (start 60 39.8278) (end 59.5278 39.8278) (width 0.2) (layer "F.Cu") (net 2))
 (segment (start 41.785 30) (end 41.285 29.5) (width 0.2) (layer "F.Cu") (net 2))
 (segment (start 31.96 52.08) (end 31.96 49.54) (width 0.2) (layer "F.Cu") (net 2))
 (segment (start 31.96 47) (end 31.96 49.54) (width 0.2) (layer "F.Cu") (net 2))
 (segment (start 53.238 32.749999) (end 52.250001 32.749999) (width 0.2) (layer "F.Cu") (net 2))
 (segment (start 53.8278 50) (end 54.75 49.0778) (width 0.2) (layer "F.Cu") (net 2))
 (segment (start 52 32.5) (end 52 33) (width 0.2) (layer "F.Cu") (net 2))
 (segment (start 54.75 49.0778) (end 54.75 47.6) (width 0.2) (layer "F.Cu") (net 2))
 (segment (start 52.25 33.25) (end 51.5 34) (width 0.2) (layer "F.Cu") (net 2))
 (segment (start 53.238 33.25) (end 53.238 32.749999) (width 0.2) (layer "F.Cu") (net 2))
 (segment (start 31.96 43) (end 31.96 44.46) (width 0.2) (layer "F.Cu") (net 2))
 (segment (start 59.5278 39.8278) (end 58.45 38.75) (width 0.2) (layer "F.Cu") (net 2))
 (segment (start 48.25 46) (end 48.25 47.6) (width 0.2) (layer "F.Cu") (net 2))
 (segment (start 31.96 34.3) (end 31.96 36.84) (width 0.2) (layer "F.Cu") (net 2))
 (segment (start 45.9 43.75) (end 46.95 43.75) (width 0.2) (layer "F.Cu") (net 2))
 (segment (start 54.2 46) (end 54.75 46.55) (width 0.2) (layer "F.Cu") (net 2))
 (segment (start 56.05 38.75) (end 57.1 38.75) (width 0.2) (layer "F.Cu") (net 2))
 (segment (start 47.739822 33.8) (end 43.851471 33.8) (width 0.2) (layer "F.Cu") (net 2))
 (segment (start 45.9 43.75) (end 44.584314 43.75) (width 0.2) (layer "F.Cu") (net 2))
 (segment (start 39.5 33) (end 39.5 29.5) (width 0.2) (layer "F.Cu") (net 2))
 (segment (start 52.25 33.25) (end 53.238 33.25) (width 0.2) (layer "F.Cu") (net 2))
 (segment (start 31.96 31.76) (end 31.96 34.3) (width 0.2) (layer "F.Cu") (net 2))
 (segment (start 41.285 29.5) (end 39.5 29.5) (width 0.2) (layer "F.Cu") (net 2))
 (segment (start 34.5 52.08) (end 31.96 52.08) (width 0.2) (layer "F.Cu") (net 2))
 (segment (start 42.8278 31.0428) (end 41.785 30) (width 0.2) (layer "F.Cu") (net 2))
 (segment (start 31.96 30.04) (end 31.96 31.76) (width 0.2) (layer "F.Cu") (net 2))
 (segment (start 32.5 29.5) (end 31.96 30.04) (width 0.2) (layer "F.Cu") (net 2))
 (segment (start 48.25 34.5778) (end 48.25 36.4) (width 0.2) (layer "F.Cu") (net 2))
 (segment (start 53.75 32.25) (end 53 31.5) (width 0.2) (layer "F.Cu") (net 2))
 (segment (start 52 33) (end 52.25 33.25) (width 0.2) (layer "F.Cu") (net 2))
 (segment (start 55.15 39.65) (end 54.9 39.9) (width 0.2) (layer "F.Cu") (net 2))
 (segment (start 54.9 39.9) (end 50.7 39.9) (width 0.2) (layer "F.Cu") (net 2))
 (segment (start 53 31.5) (end 52 32.5) (width 0.2) (layer "F.Cu") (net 2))
 (segment (start 31.96 36.84) (end 31.96 39.38) (width 0.2) (layer "F.Cu") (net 2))
 (segment (start 48.3278 34.5) (end 48.3278 33.6722) (width 0.2) (layer "F.Cu") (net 2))
 (segment (start 31.96 43) (end 38.151471 43) (width 0.2) (layer "F.Cu") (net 2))
 (segment (start 43.2278 42.9) (end 43.5 43.1722) (width 0.2) (layer "F.Cu") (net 2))
 (segment (start 50.7 39.9) (end 48.25 37.45) (width 0.2) (layer "F.Cu") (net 2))
 (segment (start 53.238 32.749999) (end 53.738001 32.749999) (width 0.2) (layer "F.Cu") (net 2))
 (segment (start 46.95 43.75) (end 48.25 45.05) (width 0.2) (layer "F.Cu") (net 2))
 (segment (start 48.3278 33.6722) (end 49 33) (width 0.2) (layer "F.Cu") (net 2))
 (segment (start 39.5 29.5) (end 32.5 29.5) (width 0.2) (layer "F.Cu") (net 2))
 (segment (start 34.5 49.54) (end 34.5 52.08) (width 0.2) (layer "F.Cu") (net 2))
 (segment (start 38.151471 43) (end 38.251471 42.9) (width 0.2) (layer "F.Cu") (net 2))
 (segment (start 31.96 41.92) (end 31.96 43) (width 0.2) (layer "F.Cu") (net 2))
 (segment (start 69 51) (end 69 51.5) (width 0.2) (layer "F.Cu") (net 2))
 (segment (start 44.006514 43.1722) (end 43.5 43.1722) (width 0.2) (layer "F.Cu") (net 2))
 (segment (start 54.75 46.55) (end 54.75 47.6) (width 0.2) (layer "F.Cu") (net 2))
 (segment (start 31.96 49.54) (end 34.5 49.54) (width 0.2) (layer "F.Cu") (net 2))
 (segment (start 54 46) (end 54.2 46) (width 0.2) (layer "F.Cu") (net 2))
 (segment (start 31.96 31.76) (end 31.96 30.96) (width 0.2) (layer "F.Cu") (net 2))
 (segment (start 54 46) (end 54 40.8) (width 0.2) (layer "F.Cu") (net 2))
 (segment (start 58.45 38.75) (end 57.1 38.75) (width 0.2) (layer "F.Cu") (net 2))
 (segment (start 52.250001 32.749999) (end 52 33) (width 0.2) (layer "F.Cu") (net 2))
 (segment (start 42.8278 34.823671) (end 42.8278 36.6722) (width 0.2) (layer "F.Cu") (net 2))
 (segment (start 31.96 39.38) (end 31.96 41.92) (width 0.2) (layer "F.Cu") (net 2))
 (segment (start 44.584314 43.75) (end 44.006514 43.1722) (width 0.2) (layer "F.Cu") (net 2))
 (segment (start 48.25 49.9222) (end 48.25 47.6) (width 0.2) (layer "F.Cu") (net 2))
 (segment (start 53.738001 32.749999) (end 53.75 32.738) (width 0.2) (layer "F.Cu") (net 2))
 (segment (start 48.3278 34.5) (end 48.25 34.5778) (width 0.2) (layer "F.Cu") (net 2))
 (segment (start 48.3278 34.5) (end 48.3278 34.387978) (width 0.2) (layer "F.Cu") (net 2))
 (segment (start 38.251471 42.9) (end 43.2278 42.9) (width 0.2) (layer "F.Cu") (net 2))
 (segment (start 43.851471 33.8) (end 42.8278 34.823671) (width 0.2) (layer "F.Cu") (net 2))
 (segment (start 55.15 39.65) (end 56.05 38.75) (width 0.2) (layer "F.Cu") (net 2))
 (segment (start 48.1722 50) (end 48.25 49.9222) (width 0.2) (layer "F.Cu") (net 2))
 (segment (start 55.6722 50) (end 54.75 49.0778) (width 0.2) (layer "F.Cu") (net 2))
 (segment (start 42.8278 36.6722) (end 42.8278 31.0428) (width 0.2) (layer "F.Cu") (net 2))
 (segment (start 48.25 45.05) (end 48.25 46) (width 0.2) (layer "F.Cu") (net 2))
 (segment (start 48.25 46) (end 54 46) (width 0.2) (layer "F.Cu") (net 2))
 (segment (start 53.75 32.738) (end 53.75 32.25) (width 0.2) (layer "F.Cu") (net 2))
 (segment (start 48.25 37.45) (end 48.25 36.4) (width 0.2) (layer "F.Cu") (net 2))
 (via (at 49 33) (size 0.6) (drill 0.3) (layers "F.Cu" "B.Cu") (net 2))
 (via (at 39.5 33) (size 0.6) (drill 0.3) (layers "F.Cu" "B.Cu") (free yes) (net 2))
 (via (at 51.5 34) (size 0.6) (drill 0.3) (layers "F.Cu" "B.Cu") (free yes) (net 2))
 (segment (start 49 33) (end 39.5 33) (width 0.2) (layer "B.Cu") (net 2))
 (segment (start 51 34) (end 50 33) (width 0.2) (layer "B.Cu") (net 2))
 (segment (start 28.5 56) (end 28.5 55.54) (width 0.2) (layer "B.Cu") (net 2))
 (segment (start 28.5 55.54) (end 31.96 52.08) (width 0.2) (layer "B.Cu") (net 2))
 (segment (start 69 51) (end 63 57) (width 0.2) (layer "B.Cu") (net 2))
 (segment (start 63 57) (end 29.5 57) (width 0.2) (layer "B.Cu") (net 2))
 (segment (start 29.5 57) (end 28.5 56) (width 0.2) (layer "B.Cu") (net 2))
 (segment (start 51.5 34) (end 51 34) (width 0.2) (layer "B.Cu") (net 2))
 (segment (start 50 33) (end 49 33) (width 0.2) (layer "B.Cu") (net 2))
 (segment (start 34.5 47) (end 36.5 45) (width 0.2) (layer "F.Cu") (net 40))
 (segment (start 61 41.5) (end 60.4 41.5) (width 0.2) (layer "F.Cu") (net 40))
 (segment (start 60.4 41.5) (end 58.15 39.25) (width 0.2) (layer "F.Cu") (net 40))
 (segment (start 36.5 45) (end 38.5 45) (width 0.2) (layer "F.Cu") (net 40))
 (segment (start 58.15 39.25) (end 57.1 39.25) (width 0.2) (layer "F.Cu") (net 40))
 (via (at 38.5 45) (size 0.6) (drill 0.3) (layers "F.Cu" "B.Cu") (free yes) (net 40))
 (via (at 61 41.5) (size 0.6) (drill 0.3) (layers "F.Cu" "B.Cu") (free yes) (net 40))
 (segment (start 39 45.5) (end 57 45.5) (width 0.2) (layer "B.Cu") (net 40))
 (segment (start 57 45.5) (end 61 41.5) (width 0.2) (layer "B.Cu") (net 40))
 (segment (start 38.5 45) (end 39 45.5) (width 0.2) (layer "B.Cu") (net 40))
 (segment (start 55.6 36.4) (end 55.25 36.4) (width 0.2) (layer "F.Cu") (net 41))
 (segment (start 34.5 44.46) (end 37.54 44.46) (width 0.2) (layer "F.Cu") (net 41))
 (segment (start 37.54 44.46) (end 38.5 43.5) (width 0.2) (layer "F.Cu") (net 41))
 (segment (start 58 34) (end 55.6 36.4) (width 0.2) (layer "F.Cu") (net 41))
 (via (at 58 34) (size 0.6) (drill 0.3) (layers "F.Cu" "B.Cu") (free yes) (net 41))
 (via (at 38.5 43.5) (size 0.6) (drill 0.3) (layers "F.Cu" "B.Cu") (free yes) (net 41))
 (segment (start 38.5 43.5) (end 48.5 43.5) (width 0.2) (layer "B.Cu") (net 41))
 (segment (start 48.5 43.5) (end 58 34) (width 0.2) (layer "B.Cu") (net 41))
 (segment (start 38.91 41.25) (end 45.9 41.25) (width 0.2) (layer "F.Cu") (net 8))
 (segment (start 34.5 36.84) (end 38.91 41.25) (width 0.2) (layer "F.Cu") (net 8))
 (segment (start 49.75 36.4) (end 49.75 33.465) (width 0.2) (layer "F.Cu") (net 52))
 (segment (start 49.75 33.465) (end 53.215 30) (width 0.2) (layer "F.Cu") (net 52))
 (segment (start 53.165686 31.1) (end 52.680686 31.1) (width 0.2) (layer "F.Cu") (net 51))
 (segment (start 52.680686 31.1) (end 50.25 33.530686) (width 0.2) (layer "F.Cu") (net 51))
 (segment (start 53.8787 31.5) (end 53.565686 31.5) (width 0.2) (layer "F.Cu") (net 51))
 (segment (start 53.565686 31.5) (end 53.165686 31.1) (width 0.2) (layer "F.Cu") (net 51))
 (segment (start 50.25 33.530686) (end 50.25 36.4) (width 0.2) (layer "F.Cu") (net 51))
 (segment (start 54.762 32.3833) (end 53.8787 31.5) (width 0.2) (layer "F.Cu") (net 51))
 (segment (start 54.762 32.749999) (end 54.762 32.3833) (width 0.2) (layer "F.Cu") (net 51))
 (segment (start 69 49) (end 66 49) (width 0.2) (layer "F.Cu") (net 36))
 (segment (start 58.25 41.25) (end 57.1 41.25) (width 0.2) (layer "F.Cu") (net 36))
 (segment (start 66 49) (end 58.25 41.25) (width 0.2) (layer "F.Cu") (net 36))
 (segment (start 51.362 34.738) (end 50.75 35.35) (width 0.2) (layer "F.Cu") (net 50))
 (segment (start 50.75 35.35) (end 50.75 36.4) (width 0.2) (layer "F.Cu") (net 50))
 (segment (start 54.762 34.738) (end 51.362 34.738) (width 0.2) (layer "F.Cu") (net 50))
 (segment (start 54.762 34.250001) (end 54.762 34.738) (width 0.2) (layer "F.Cu") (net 50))
 (segment (start 69 47) (end 64.5 42.5) (width 0.2) (layer "F.Cu") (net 37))
 (segment (start 60.834314 42.5) (end 59.084314 40.75) (width 0.2) (layer "F.Cu") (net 37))
 (segment (start 59.084314 40.75) (end 57.1 40.75) (width 0.2) (layer "F.Cu") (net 37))
 (segment (start 64.5 42.5) (end 60.834314 42.5) (width 0.2) (layer "F.Cu") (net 37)))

